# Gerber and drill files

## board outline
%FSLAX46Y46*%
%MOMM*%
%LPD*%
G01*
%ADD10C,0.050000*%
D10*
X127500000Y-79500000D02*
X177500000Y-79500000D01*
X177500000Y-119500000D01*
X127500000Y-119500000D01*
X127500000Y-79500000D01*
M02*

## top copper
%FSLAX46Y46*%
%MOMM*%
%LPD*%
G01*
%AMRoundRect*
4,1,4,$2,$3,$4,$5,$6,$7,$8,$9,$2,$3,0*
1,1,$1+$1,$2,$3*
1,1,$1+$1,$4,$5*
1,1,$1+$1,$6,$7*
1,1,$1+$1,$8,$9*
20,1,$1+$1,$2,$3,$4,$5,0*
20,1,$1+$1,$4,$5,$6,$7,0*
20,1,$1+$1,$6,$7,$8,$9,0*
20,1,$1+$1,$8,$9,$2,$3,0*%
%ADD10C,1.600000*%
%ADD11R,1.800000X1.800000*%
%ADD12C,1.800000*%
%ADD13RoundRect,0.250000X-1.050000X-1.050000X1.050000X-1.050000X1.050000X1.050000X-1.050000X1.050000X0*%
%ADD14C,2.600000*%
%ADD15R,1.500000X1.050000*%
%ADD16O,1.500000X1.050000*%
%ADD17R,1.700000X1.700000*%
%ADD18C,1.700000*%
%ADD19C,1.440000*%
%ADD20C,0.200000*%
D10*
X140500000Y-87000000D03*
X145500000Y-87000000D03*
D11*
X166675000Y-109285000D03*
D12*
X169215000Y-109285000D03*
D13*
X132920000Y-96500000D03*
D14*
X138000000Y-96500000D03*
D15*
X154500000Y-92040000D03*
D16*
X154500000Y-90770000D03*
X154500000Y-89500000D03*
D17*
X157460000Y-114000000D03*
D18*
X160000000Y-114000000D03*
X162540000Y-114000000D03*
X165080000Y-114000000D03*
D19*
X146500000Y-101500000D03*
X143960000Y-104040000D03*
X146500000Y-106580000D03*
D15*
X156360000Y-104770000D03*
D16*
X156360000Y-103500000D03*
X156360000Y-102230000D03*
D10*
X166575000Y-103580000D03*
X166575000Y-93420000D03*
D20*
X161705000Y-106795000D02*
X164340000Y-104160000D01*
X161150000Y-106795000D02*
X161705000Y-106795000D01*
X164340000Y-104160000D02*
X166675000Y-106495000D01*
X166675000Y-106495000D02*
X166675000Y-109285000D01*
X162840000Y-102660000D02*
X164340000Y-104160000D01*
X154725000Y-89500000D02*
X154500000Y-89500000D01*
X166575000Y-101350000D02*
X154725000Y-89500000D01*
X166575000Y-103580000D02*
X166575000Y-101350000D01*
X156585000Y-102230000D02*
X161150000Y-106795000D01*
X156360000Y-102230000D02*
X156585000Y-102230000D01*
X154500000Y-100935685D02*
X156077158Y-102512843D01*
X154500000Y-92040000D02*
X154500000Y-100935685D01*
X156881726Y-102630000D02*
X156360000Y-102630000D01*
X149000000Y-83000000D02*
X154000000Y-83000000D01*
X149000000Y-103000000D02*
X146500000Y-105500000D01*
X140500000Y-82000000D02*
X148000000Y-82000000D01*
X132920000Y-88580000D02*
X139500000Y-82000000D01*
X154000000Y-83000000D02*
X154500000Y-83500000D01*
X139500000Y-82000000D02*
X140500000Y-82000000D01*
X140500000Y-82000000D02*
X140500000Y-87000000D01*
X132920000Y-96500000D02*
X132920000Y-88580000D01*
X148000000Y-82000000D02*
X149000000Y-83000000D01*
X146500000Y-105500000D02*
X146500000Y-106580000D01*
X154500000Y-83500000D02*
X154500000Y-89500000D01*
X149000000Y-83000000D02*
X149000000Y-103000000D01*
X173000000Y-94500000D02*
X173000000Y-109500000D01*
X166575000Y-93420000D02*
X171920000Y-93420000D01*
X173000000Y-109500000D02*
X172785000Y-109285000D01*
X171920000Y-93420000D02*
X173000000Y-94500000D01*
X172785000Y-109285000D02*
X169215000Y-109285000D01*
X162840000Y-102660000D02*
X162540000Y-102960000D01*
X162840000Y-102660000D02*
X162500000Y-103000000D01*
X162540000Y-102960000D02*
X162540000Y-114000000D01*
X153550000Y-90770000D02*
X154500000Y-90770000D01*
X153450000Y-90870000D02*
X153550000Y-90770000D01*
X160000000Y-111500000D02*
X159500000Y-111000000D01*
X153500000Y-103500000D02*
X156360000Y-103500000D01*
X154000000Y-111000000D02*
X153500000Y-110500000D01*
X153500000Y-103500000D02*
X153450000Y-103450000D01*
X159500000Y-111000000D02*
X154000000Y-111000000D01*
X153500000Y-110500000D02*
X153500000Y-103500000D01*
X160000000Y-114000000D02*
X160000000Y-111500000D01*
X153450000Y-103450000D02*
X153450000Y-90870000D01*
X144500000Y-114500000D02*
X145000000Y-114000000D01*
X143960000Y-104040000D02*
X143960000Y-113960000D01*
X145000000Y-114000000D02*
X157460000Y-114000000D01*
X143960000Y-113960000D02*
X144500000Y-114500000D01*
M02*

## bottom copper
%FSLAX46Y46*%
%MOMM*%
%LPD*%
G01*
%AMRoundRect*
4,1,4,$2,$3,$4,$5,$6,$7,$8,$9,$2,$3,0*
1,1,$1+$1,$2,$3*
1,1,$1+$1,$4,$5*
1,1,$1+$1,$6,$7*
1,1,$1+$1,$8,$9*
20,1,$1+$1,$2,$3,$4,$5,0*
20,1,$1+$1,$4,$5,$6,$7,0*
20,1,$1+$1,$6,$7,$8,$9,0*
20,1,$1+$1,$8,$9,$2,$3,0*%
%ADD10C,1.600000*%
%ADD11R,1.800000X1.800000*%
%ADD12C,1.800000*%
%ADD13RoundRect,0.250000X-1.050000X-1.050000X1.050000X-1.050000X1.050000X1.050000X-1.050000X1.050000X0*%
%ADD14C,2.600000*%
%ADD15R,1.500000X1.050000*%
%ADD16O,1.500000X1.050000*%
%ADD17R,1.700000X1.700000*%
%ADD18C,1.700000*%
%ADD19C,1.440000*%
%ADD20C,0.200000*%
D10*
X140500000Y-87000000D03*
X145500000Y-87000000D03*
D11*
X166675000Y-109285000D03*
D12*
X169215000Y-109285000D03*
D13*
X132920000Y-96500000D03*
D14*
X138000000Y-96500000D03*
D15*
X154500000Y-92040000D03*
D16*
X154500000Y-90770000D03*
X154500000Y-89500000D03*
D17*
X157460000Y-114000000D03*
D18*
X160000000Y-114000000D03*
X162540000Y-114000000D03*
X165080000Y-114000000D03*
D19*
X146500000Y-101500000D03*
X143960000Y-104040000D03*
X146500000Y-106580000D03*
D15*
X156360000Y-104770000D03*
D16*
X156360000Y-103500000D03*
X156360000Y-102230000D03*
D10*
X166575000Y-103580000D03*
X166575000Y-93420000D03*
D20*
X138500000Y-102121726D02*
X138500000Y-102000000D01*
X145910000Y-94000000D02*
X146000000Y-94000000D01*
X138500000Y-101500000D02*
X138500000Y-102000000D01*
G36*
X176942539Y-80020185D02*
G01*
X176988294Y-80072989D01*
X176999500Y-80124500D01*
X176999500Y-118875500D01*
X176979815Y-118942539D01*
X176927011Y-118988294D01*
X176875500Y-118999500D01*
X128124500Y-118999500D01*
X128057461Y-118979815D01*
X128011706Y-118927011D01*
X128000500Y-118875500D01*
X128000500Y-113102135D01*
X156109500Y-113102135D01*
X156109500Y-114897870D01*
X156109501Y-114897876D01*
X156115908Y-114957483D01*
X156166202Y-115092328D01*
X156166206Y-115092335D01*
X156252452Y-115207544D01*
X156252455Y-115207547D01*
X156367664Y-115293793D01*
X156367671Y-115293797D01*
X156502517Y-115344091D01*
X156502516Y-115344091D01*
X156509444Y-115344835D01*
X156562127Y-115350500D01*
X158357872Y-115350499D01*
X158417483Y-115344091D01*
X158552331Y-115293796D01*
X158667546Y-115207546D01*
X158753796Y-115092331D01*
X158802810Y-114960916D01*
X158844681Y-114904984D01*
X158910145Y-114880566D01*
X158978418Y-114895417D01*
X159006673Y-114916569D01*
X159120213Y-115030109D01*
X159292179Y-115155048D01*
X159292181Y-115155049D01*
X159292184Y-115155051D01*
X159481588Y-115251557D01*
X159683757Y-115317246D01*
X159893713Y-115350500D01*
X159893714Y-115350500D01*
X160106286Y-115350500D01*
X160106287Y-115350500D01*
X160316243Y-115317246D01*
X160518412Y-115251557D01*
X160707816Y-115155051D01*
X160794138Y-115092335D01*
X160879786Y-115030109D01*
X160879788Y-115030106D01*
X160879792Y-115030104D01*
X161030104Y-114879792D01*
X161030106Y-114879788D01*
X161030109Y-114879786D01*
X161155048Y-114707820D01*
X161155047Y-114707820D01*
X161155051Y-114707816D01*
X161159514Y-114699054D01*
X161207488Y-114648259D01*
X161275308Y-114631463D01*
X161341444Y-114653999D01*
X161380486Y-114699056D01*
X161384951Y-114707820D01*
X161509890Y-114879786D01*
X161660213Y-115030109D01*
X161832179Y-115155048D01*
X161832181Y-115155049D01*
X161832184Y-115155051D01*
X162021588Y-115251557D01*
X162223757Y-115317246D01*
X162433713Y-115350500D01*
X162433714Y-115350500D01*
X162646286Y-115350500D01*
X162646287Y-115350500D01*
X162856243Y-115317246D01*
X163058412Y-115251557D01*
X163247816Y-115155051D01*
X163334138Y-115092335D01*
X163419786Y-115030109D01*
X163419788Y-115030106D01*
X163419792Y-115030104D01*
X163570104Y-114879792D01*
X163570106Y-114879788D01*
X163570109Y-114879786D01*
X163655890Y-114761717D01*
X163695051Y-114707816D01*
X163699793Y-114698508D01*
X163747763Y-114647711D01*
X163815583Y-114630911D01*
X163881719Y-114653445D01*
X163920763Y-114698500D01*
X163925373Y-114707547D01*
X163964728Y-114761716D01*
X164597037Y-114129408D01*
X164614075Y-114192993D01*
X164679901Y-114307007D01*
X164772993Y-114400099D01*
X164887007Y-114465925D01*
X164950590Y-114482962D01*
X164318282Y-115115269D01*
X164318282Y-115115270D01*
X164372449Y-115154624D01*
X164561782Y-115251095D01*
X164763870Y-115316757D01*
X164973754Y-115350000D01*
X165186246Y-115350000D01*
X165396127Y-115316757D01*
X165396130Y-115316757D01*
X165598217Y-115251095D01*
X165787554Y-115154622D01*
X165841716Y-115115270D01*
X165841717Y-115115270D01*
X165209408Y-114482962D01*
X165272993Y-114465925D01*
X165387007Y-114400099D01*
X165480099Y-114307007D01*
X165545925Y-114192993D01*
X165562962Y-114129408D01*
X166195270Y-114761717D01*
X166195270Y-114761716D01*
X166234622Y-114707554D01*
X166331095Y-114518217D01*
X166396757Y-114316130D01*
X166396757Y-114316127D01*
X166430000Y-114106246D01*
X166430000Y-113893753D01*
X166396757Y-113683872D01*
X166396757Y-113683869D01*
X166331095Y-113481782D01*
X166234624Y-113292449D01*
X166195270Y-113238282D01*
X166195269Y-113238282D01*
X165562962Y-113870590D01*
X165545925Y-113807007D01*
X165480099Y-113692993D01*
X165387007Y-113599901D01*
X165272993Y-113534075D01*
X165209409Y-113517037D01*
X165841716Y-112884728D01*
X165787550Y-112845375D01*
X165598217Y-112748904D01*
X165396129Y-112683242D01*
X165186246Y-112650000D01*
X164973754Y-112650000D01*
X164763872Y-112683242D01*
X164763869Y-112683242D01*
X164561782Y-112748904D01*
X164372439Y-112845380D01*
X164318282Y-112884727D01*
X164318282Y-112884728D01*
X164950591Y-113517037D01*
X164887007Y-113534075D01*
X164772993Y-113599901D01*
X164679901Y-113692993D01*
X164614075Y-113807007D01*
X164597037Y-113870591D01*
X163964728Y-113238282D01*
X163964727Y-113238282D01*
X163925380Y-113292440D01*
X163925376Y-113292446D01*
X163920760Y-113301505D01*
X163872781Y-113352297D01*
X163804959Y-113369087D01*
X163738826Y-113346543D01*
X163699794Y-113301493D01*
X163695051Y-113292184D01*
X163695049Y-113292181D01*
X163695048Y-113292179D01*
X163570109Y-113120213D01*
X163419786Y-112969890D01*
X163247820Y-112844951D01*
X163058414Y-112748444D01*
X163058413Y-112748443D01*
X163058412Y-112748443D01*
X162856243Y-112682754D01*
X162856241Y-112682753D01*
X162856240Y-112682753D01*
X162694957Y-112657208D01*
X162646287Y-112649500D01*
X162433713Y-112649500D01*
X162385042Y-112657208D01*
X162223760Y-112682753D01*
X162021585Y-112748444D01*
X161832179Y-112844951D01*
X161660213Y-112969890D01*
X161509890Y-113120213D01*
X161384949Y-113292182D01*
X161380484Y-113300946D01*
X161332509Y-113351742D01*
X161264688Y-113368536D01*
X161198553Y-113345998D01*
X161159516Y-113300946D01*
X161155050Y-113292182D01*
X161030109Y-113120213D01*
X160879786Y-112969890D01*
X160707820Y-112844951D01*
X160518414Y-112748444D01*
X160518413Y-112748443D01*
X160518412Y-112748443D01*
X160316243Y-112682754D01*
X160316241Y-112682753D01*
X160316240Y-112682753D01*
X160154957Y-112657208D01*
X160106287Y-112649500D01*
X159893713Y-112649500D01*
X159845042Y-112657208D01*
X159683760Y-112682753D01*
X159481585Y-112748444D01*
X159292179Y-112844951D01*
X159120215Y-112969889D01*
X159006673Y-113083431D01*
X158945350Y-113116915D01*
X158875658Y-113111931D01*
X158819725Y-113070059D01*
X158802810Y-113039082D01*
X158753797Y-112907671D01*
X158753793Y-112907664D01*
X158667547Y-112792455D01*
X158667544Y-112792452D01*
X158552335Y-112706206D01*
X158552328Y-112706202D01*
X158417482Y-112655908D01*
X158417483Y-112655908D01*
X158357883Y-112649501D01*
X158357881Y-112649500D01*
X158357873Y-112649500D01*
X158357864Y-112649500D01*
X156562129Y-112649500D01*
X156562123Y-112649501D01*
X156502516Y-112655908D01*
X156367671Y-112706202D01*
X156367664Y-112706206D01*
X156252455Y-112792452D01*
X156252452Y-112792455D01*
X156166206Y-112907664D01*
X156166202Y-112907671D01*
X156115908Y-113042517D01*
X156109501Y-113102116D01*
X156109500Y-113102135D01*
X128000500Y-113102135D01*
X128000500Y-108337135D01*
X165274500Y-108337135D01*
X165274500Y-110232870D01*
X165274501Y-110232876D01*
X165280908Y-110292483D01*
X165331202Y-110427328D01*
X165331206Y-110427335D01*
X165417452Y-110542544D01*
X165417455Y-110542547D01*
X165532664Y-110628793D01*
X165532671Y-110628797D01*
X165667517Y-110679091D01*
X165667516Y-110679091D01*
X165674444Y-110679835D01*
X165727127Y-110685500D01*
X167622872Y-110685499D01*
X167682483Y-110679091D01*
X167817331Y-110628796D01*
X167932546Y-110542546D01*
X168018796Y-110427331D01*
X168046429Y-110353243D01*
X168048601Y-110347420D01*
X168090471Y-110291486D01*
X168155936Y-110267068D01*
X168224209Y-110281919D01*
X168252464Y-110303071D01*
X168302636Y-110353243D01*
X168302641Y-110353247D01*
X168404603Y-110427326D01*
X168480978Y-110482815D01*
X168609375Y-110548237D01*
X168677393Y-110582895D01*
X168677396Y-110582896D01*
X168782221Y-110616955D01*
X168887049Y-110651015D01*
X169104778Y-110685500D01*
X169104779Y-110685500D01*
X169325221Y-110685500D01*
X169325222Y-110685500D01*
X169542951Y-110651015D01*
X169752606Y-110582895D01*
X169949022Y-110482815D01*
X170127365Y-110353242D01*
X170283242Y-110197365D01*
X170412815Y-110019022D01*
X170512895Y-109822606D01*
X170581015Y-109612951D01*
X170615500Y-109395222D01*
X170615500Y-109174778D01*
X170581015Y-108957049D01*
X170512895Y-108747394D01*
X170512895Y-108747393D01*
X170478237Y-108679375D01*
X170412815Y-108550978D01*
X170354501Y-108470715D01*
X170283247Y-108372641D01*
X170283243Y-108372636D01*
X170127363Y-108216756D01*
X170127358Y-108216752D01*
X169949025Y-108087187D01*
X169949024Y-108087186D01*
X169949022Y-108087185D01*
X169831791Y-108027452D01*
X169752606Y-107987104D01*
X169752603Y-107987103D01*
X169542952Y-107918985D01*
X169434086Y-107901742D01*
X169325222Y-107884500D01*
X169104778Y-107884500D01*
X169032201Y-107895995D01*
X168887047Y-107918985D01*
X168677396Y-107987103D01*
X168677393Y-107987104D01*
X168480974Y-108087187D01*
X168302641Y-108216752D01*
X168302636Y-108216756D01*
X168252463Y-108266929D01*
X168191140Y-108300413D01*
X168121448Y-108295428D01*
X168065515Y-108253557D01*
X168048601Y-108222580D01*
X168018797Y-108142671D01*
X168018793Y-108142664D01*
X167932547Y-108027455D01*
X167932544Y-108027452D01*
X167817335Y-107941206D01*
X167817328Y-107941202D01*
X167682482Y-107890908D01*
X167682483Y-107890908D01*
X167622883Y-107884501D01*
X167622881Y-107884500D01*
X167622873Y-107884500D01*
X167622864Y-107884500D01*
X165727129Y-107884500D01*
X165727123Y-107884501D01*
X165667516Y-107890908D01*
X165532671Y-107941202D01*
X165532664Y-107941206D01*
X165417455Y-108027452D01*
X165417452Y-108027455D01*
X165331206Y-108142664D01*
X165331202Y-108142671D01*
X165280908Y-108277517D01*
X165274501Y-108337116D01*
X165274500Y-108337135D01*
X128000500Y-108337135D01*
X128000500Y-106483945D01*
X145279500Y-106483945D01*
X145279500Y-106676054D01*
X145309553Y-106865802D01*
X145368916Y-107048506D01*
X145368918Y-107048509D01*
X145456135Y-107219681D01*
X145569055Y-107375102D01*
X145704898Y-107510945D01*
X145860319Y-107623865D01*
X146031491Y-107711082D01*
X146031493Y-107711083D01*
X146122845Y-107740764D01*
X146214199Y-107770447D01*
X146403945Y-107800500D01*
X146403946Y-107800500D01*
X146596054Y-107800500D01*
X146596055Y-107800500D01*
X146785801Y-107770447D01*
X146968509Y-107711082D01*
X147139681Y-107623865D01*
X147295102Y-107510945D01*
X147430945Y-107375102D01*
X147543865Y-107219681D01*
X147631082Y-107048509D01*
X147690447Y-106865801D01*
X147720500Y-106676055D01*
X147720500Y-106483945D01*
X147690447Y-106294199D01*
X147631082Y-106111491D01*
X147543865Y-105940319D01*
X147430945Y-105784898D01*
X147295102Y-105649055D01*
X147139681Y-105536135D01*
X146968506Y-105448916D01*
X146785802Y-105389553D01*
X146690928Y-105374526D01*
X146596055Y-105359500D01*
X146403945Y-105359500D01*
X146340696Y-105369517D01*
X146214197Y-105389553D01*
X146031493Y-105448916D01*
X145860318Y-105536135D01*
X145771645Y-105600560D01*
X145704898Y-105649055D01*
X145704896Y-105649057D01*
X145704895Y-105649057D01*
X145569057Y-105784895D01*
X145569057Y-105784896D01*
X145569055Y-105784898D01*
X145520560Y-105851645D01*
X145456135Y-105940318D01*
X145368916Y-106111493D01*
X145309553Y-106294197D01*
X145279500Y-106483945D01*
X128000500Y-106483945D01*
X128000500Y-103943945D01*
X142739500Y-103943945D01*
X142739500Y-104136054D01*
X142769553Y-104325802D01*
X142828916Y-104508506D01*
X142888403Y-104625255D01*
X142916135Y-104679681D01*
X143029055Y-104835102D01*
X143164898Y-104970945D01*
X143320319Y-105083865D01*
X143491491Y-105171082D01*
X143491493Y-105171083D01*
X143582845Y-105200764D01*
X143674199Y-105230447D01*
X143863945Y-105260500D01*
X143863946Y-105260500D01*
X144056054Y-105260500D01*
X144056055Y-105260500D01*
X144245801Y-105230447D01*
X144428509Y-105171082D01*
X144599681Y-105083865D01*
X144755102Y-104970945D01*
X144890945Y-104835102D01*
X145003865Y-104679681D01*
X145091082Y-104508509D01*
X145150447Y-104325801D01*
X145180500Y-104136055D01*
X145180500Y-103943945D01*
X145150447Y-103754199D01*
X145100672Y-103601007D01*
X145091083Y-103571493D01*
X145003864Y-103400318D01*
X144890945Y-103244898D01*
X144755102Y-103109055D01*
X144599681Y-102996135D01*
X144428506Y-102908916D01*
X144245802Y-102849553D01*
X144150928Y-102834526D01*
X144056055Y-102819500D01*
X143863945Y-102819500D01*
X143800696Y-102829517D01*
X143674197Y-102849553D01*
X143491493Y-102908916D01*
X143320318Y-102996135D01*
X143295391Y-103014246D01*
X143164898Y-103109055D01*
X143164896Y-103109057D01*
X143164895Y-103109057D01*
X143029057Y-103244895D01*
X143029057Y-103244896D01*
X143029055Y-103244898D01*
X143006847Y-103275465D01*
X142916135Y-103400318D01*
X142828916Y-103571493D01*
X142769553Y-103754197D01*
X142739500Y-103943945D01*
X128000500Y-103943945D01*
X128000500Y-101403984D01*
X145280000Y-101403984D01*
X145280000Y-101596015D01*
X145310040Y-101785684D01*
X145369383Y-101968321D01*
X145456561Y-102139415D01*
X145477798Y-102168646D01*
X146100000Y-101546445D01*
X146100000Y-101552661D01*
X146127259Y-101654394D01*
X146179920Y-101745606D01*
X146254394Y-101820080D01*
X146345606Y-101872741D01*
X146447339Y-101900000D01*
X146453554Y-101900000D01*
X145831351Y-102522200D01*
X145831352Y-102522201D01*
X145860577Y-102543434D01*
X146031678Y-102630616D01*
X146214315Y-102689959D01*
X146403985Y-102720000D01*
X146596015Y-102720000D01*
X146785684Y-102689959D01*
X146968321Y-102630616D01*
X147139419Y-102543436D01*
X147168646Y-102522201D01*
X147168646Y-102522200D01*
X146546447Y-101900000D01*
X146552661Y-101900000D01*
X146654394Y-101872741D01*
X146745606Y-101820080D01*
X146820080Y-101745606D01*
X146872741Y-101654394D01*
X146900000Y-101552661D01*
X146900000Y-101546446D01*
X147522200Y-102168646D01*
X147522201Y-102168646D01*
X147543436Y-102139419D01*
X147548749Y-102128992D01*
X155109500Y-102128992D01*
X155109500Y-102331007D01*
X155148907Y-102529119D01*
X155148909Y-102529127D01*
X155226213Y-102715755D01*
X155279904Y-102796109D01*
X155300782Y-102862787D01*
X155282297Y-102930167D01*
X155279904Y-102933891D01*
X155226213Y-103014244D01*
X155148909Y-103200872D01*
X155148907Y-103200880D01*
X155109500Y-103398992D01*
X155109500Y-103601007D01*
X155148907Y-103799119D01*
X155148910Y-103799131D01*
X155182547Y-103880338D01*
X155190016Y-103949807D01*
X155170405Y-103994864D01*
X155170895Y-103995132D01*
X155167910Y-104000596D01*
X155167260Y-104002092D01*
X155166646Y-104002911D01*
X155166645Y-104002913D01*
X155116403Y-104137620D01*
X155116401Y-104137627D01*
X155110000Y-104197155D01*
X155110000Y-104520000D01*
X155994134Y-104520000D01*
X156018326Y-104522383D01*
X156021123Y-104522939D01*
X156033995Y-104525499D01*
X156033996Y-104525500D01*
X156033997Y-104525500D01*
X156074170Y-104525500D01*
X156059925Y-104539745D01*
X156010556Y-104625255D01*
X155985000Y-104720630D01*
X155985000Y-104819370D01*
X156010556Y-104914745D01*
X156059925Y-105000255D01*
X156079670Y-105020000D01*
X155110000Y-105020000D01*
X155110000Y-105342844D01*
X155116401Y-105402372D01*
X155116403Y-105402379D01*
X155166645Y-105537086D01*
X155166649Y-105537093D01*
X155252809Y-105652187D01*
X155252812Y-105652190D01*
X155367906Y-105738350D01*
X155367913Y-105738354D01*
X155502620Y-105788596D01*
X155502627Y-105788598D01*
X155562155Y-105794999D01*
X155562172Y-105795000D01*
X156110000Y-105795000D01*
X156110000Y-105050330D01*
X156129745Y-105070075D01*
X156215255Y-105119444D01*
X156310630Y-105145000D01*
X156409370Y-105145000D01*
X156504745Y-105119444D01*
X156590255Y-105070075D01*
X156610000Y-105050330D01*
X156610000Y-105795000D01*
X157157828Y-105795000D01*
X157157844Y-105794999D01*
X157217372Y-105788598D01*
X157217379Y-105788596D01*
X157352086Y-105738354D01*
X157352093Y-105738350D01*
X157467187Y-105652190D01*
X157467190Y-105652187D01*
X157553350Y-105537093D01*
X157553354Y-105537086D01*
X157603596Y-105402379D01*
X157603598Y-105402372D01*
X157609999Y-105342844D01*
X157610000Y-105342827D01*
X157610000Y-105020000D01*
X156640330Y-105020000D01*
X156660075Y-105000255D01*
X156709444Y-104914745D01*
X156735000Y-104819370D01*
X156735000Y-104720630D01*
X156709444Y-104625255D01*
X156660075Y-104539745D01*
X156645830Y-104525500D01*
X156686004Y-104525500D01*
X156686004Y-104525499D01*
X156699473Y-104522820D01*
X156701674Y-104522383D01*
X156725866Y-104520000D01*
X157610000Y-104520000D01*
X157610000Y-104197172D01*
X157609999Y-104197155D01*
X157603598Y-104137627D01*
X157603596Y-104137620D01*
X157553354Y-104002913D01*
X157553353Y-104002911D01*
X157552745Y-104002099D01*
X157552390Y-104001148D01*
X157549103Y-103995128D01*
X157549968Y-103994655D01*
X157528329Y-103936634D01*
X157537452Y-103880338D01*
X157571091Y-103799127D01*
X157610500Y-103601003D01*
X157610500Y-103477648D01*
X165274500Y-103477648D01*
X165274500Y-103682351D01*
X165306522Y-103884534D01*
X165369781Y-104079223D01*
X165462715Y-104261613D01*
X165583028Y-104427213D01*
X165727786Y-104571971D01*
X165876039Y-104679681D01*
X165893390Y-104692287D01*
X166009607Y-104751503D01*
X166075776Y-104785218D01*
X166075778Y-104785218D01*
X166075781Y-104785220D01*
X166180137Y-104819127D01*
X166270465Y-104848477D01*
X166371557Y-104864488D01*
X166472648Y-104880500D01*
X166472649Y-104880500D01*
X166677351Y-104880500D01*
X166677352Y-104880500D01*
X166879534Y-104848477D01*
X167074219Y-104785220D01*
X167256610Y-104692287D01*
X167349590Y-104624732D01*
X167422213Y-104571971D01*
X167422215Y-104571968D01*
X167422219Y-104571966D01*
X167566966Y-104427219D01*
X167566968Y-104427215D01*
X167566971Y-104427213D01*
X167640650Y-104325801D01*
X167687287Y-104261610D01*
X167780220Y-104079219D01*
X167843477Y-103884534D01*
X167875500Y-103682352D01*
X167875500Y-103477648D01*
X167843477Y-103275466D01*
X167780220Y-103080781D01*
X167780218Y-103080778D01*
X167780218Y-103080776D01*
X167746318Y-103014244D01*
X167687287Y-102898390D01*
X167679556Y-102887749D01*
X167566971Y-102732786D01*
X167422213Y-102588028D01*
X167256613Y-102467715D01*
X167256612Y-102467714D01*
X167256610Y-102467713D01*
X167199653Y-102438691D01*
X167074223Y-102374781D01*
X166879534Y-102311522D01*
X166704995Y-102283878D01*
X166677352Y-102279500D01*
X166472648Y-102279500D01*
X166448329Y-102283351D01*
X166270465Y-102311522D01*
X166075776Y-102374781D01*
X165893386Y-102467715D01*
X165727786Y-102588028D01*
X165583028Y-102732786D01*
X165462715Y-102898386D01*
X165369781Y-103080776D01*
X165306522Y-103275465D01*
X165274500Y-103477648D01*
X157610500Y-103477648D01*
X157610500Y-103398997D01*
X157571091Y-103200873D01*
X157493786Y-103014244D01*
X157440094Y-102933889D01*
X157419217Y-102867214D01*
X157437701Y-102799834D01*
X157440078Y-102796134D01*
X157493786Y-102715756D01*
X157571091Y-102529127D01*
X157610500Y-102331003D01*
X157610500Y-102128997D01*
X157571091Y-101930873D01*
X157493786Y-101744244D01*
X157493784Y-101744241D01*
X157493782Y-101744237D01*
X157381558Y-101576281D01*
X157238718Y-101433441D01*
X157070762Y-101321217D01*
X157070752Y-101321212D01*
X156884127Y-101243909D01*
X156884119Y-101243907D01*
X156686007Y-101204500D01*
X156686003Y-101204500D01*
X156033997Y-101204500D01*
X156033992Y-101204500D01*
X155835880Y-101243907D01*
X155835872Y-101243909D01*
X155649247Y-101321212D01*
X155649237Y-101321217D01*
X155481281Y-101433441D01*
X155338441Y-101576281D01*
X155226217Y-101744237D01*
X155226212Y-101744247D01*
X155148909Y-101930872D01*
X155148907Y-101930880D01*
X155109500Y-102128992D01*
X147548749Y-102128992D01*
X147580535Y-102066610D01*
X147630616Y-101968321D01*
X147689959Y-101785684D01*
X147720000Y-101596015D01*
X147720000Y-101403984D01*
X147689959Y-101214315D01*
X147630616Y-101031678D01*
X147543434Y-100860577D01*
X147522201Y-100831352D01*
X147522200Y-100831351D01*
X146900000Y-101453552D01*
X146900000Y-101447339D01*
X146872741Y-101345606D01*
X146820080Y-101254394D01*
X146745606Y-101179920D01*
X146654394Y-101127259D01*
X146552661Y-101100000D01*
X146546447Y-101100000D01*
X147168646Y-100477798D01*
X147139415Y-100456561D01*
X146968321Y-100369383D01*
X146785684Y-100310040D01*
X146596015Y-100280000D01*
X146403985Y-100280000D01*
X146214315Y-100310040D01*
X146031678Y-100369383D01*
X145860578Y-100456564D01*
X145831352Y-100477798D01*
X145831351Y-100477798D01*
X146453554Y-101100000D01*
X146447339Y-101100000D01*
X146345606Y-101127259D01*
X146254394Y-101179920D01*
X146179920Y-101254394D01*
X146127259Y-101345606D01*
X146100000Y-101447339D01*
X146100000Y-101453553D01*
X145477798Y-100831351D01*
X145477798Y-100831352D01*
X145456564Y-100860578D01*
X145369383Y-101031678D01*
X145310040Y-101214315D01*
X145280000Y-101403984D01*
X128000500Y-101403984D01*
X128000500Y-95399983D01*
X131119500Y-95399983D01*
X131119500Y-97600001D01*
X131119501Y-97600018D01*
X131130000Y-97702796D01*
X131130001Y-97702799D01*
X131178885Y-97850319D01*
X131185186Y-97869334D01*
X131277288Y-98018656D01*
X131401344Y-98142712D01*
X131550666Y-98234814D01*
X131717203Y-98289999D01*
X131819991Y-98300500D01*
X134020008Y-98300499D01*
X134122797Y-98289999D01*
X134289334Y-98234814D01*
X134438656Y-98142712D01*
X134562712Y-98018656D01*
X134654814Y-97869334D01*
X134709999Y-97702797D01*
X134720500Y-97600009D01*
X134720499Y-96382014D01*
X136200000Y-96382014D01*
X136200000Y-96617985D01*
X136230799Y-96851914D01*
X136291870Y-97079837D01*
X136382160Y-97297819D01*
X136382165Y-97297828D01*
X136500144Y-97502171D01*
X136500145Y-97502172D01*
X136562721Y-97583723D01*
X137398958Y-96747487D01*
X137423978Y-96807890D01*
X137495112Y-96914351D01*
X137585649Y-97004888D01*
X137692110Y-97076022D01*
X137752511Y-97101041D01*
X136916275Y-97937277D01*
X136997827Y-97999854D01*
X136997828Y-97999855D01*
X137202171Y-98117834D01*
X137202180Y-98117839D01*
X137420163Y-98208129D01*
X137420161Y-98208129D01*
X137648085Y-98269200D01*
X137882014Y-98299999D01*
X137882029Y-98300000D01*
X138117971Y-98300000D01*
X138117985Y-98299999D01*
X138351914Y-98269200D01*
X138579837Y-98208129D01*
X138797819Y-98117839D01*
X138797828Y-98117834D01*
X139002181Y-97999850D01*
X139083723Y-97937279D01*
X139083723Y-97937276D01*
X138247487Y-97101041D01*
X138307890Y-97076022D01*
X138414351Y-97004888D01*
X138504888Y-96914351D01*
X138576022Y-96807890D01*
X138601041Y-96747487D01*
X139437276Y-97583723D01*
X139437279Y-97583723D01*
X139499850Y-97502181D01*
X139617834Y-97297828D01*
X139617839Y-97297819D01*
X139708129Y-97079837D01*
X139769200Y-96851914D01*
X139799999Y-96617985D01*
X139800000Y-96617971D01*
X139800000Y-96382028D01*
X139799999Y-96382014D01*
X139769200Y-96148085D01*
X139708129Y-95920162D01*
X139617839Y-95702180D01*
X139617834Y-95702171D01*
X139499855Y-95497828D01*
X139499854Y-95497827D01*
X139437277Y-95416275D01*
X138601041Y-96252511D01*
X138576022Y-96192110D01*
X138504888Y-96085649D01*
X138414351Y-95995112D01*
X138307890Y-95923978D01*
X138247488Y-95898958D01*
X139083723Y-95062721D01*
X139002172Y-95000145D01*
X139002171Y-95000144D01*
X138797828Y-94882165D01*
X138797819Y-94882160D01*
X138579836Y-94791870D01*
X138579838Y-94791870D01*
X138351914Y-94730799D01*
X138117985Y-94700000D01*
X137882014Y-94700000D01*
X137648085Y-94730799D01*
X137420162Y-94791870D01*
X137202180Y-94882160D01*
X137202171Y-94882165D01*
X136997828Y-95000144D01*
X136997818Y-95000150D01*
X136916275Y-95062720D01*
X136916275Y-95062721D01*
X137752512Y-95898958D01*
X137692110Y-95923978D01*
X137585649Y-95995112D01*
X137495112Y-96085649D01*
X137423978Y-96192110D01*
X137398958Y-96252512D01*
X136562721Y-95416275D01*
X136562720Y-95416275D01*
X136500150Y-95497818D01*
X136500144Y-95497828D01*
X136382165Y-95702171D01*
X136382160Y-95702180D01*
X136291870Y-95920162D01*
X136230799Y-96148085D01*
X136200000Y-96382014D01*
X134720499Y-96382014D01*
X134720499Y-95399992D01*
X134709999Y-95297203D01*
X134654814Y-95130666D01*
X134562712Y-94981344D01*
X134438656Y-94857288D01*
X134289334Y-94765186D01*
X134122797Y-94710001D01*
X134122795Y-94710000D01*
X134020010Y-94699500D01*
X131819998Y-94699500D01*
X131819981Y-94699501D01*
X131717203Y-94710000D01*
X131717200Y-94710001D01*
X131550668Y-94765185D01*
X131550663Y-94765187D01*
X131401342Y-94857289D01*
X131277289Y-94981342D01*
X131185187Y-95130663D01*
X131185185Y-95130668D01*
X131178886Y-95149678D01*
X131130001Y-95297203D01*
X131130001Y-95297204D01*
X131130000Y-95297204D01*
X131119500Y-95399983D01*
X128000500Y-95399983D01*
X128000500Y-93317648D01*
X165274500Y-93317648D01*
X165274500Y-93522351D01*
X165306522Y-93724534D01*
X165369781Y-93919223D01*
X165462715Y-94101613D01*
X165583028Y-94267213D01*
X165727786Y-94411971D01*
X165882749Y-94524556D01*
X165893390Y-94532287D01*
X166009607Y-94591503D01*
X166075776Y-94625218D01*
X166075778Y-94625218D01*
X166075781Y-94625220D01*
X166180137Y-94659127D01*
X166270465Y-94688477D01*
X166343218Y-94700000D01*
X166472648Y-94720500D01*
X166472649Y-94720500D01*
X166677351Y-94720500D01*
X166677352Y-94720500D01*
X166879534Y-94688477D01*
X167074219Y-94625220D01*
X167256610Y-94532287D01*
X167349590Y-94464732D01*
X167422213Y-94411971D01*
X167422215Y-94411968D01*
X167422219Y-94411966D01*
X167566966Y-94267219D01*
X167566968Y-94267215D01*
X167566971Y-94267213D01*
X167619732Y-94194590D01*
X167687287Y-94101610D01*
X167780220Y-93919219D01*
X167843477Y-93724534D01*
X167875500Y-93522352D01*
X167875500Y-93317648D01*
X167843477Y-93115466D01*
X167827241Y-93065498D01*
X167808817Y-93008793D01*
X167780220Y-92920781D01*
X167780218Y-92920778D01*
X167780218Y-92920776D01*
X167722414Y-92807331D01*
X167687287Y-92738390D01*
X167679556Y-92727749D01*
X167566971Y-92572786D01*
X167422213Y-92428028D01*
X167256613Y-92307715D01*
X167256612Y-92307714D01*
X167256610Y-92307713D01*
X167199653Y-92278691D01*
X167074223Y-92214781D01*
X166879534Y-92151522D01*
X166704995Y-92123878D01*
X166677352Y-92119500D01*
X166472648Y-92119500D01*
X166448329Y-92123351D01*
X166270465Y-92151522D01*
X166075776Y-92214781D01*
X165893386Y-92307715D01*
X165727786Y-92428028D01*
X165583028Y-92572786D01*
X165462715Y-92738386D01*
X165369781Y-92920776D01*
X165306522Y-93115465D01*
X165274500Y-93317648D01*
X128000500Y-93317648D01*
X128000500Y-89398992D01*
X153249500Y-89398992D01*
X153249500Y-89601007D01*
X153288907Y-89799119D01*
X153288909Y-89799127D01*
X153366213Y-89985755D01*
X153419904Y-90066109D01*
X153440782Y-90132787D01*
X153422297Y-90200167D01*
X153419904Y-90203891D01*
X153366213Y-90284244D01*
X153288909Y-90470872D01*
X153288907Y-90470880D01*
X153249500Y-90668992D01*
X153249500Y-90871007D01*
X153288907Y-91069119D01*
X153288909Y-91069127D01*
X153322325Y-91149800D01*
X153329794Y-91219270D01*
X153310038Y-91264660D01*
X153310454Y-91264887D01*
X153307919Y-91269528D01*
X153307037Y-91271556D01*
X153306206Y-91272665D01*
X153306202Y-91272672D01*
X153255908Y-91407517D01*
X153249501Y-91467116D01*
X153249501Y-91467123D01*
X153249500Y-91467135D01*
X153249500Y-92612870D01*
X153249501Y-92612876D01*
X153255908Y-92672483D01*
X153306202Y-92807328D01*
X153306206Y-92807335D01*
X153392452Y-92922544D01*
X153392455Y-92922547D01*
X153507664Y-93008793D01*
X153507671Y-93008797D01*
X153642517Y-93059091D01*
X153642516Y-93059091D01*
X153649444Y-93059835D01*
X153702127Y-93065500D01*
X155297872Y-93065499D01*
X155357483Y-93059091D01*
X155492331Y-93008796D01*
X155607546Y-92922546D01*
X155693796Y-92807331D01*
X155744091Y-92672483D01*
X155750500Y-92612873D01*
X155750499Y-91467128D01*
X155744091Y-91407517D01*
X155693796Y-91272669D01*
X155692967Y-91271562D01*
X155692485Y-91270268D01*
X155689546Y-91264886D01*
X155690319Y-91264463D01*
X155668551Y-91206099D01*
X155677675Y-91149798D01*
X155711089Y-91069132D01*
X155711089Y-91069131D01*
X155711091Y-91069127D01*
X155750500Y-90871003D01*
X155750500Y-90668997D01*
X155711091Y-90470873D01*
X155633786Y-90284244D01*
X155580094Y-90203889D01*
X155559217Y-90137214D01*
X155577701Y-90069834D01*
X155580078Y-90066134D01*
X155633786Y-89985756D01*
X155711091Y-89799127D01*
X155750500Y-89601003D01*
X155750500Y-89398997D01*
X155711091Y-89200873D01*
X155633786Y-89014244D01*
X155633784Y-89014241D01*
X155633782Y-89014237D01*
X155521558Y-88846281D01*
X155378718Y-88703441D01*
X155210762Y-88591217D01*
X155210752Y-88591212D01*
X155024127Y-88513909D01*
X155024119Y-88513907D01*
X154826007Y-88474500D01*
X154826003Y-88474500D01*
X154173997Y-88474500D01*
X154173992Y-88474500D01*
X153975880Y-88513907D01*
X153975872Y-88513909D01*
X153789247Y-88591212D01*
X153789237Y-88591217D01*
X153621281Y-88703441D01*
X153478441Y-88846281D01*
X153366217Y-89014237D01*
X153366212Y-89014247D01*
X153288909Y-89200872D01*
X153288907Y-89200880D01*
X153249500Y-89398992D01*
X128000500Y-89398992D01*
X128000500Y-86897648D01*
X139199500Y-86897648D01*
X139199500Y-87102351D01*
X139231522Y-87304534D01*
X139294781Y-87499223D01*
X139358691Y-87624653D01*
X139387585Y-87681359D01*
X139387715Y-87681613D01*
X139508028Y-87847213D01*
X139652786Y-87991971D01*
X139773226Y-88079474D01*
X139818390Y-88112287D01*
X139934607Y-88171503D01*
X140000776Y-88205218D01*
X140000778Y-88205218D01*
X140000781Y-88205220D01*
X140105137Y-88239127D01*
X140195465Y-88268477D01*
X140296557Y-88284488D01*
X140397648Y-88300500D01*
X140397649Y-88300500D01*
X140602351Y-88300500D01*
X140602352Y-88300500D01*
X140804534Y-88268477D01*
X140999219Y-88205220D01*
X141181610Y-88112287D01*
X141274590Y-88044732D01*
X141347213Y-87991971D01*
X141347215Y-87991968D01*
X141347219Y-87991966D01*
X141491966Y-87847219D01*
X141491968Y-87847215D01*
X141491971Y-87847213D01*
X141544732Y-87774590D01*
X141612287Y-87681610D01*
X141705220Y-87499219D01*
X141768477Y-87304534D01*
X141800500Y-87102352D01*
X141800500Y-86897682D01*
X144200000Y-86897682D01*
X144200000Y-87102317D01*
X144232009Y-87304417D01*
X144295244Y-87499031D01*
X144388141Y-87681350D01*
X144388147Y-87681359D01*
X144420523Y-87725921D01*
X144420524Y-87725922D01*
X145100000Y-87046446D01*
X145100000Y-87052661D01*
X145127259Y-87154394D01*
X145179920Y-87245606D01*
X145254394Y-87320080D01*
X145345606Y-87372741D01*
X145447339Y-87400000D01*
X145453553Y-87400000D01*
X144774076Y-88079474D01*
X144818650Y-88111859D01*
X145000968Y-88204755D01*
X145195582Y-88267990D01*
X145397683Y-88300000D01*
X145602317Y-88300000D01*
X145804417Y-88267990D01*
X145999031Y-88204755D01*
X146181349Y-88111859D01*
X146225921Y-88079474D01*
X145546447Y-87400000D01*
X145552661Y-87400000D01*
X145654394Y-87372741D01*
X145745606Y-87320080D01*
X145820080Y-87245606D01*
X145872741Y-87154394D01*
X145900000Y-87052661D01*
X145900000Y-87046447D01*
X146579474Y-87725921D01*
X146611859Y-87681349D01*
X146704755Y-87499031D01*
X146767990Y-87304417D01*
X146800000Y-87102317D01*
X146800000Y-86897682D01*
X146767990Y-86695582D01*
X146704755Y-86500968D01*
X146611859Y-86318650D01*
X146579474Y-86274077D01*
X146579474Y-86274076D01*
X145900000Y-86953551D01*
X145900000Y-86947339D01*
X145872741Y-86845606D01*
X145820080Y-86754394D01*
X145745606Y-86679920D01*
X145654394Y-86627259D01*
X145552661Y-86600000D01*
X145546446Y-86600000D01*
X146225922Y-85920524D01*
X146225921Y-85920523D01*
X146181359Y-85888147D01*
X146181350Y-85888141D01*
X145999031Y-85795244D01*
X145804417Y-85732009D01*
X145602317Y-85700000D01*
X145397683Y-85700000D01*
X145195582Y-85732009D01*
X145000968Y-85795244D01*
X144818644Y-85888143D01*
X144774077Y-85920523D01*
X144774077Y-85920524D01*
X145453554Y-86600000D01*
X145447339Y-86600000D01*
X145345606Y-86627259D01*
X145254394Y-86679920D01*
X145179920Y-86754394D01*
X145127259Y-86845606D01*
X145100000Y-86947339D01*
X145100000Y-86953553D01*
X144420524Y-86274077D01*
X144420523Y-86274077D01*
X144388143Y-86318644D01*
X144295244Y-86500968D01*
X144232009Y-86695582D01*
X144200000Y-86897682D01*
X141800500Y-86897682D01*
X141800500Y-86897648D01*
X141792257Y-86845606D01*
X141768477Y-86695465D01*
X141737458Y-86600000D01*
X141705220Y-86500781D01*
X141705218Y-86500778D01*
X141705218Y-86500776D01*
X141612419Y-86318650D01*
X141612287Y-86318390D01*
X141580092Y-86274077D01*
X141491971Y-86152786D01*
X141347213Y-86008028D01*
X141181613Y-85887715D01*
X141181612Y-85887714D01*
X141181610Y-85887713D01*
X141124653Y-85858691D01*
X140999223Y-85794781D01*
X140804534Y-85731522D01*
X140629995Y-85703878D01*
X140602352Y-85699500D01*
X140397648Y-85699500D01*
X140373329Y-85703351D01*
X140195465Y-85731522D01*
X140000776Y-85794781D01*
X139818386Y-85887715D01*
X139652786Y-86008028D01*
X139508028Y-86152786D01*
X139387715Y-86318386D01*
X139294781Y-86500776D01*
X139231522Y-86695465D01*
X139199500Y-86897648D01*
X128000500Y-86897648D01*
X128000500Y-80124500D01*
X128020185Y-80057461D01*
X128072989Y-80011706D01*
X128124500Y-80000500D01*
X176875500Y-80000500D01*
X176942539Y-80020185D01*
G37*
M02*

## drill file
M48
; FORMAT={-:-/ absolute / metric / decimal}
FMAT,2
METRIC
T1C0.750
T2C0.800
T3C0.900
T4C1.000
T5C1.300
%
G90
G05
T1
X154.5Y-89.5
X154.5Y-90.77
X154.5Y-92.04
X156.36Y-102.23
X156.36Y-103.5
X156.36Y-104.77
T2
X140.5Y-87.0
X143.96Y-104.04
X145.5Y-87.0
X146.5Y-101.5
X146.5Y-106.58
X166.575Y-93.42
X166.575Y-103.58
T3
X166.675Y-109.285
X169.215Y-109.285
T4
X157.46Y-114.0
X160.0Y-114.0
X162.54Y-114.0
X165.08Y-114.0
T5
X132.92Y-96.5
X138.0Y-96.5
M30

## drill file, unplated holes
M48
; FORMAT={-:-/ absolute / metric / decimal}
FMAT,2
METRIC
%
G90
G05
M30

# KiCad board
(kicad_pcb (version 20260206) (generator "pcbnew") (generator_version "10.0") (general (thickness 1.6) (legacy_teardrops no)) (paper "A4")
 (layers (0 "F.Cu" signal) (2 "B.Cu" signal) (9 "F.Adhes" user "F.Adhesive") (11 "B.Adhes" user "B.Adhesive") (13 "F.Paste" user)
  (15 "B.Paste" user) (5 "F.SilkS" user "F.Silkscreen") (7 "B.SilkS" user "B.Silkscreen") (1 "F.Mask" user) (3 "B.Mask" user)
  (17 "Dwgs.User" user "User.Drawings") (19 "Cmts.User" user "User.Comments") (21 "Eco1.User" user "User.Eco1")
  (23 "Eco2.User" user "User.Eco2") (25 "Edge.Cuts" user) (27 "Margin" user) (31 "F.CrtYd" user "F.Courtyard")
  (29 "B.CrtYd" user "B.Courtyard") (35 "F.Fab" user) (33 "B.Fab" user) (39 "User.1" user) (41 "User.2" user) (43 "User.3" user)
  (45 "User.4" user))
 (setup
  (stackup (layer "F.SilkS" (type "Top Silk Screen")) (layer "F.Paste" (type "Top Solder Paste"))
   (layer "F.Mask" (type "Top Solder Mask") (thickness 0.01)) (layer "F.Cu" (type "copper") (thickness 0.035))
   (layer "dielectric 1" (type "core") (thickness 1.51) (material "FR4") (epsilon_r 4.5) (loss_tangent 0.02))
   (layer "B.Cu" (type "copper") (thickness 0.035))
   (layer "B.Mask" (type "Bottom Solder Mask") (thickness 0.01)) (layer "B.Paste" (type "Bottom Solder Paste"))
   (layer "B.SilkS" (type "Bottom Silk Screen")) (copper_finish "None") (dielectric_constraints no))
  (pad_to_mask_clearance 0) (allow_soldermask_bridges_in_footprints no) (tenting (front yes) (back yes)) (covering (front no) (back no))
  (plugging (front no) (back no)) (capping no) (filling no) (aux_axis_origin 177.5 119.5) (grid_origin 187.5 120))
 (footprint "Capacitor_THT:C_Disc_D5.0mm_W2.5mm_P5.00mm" (layer "F.Cu") (at 140.5 87)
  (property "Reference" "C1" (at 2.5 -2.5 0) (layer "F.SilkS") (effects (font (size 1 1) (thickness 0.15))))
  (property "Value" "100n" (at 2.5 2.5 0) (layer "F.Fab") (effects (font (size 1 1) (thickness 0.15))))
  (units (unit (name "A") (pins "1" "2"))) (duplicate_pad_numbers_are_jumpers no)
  (pad "1" thru_hole circle (at 0 0) (size 1.6 1.6) (drill 0.8) (layers "*.Cu" "*.Mask") (remove_unused_layers no) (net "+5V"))
  (pad "2" thru_hole circle (at 5 0) (size 1.6 1.6) (drill 0.8) (layers "*.Cu" "*.Mask") (remove_unused_layers no) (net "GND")))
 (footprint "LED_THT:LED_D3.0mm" (layer "F.Cu") (at 166.675 109.285)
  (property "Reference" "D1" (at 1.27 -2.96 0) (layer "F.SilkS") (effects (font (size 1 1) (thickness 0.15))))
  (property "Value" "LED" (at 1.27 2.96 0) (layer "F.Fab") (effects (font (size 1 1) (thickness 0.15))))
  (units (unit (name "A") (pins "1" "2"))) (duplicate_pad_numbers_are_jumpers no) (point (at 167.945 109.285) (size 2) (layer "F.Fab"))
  (pad "1" thru_hole rect (at 0 0) (size 1.8 1.8) (drill 0.9) (layers "*.Cu" "*.Mask") (remove_unused_layers no) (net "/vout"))
  (pad "2" thru_hole circle (at 2.54 0) (size 1.8 1.8) (drill 0.9) (layers "*.Cu" "*.Mask") (remove_unused_layers no) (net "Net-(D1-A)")))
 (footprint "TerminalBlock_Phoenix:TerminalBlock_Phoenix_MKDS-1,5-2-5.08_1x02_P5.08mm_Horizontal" (layer "F.Cu") (at 132.92 96.5)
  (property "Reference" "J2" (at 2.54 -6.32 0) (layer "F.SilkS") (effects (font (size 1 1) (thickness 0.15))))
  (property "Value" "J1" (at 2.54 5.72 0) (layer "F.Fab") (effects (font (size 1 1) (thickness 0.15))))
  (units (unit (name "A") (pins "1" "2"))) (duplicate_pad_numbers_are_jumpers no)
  (pad "1" thru_hole roundrect (at 0 0) (size 2.6 2.6) (drill 1.3) (layers "*.Cu" "*.Mask") (remove_unused_layers no)
   (roundrect_rratio 0.096154) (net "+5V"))
  (pad "2" thru_hole circle (at 5.08 0) (size 2.6 2.6) (drill 1.3) (layers "*.Cu" "*.Mask") (remove_unused_layers no) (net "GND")))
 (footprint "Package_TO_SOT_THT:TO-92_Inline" (layer "F.Cu") (at 154.5 92.04 90)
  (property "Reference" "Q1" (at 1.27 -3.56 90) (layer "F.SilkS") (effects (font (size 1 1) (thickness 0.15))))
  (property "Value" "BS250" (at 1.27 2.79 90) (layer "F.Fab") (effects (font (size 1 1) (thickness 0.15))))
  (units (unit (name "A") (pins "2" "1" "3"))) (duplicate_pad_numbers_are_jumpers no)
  (pad "1" thru_hole rect (at 0 0 90) (size 1.05 1.5) (drill 0.75) (layers "*.Cu" "*.Mask") (remove_unused_layers no) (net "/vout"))
  (pad "2" thru_hole oval (at 1.27 0 90) (size 1.05 1.5) (drill 0.75) (layers "*.Cu" "*.Mask") (remove_unused_layers no) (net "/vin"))
  (pad "3" thru_hole oval (at 2.54 0 90) (size 1.05 1.5) (drill 0.75) (layers "*.Cu" "*.Mask") (remove_unused_layers no) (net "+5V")))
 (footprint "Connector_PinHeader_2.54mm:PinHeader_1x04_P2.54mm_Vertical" (layer "F.Cu") (at 157.46 114 90)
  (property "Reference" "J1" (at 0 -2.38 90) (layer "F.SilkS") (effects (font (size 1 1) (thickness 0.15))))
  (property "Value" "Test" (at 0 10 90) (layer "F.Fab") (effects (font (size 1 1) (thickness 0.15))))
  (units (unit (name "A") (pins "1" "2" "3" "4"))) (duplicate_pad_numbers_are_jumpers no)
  (pad "1" thru_hole rect (at 0 0 90) (size 1.7 1.7) (drill 1) (layers "*.Cu" "*.Mask") (remove_unused_layers no) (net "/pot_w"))
  (pad "2" thru_hole circle (at 0 2.54 90) (size 1.7 1.7) (drill 1) (layers "*.Cu" "*.Mask") (remove_unused_layers no) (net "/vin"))
  (pad "3" thru_hole circle (at 0 5.08 90) (size 1.7 1.7) (drill 1) (layers "*.Cu" "*.Mask") (remove_unused_layers no) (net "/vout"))
  (pad "4" thru_hole circle (at 0 7.62 90) (size 1.7 1.7) (drill 1) (layers "*.Cu" "*.Mask") (remove_unused_layers no) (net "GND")))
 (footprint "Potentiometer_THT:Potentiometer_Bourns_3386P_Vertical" (layer "F.Cu") (at 146.5 101.5 180)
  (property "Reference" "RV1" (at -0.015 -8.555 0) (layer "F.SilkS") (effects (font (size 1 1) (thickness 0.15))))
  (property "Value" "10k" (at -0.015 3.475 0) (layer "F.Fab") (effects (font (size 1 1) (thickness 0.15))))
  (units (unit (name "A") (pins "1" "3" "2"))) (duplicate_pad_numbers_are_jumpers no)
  (pad "1" thru_hole circle (at 0 0 180) (size 1.44 1.44) (drill 0.8) (layers "*.Cu" "*.Mask") (remove_unused_layers no) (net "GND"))
  (pad "2" thru_hole circle (at 2.54 -2.54 180) (size 1.44 1.44) (drill 0.8) (layers "*.Cu" "*.Mask") (remove_unused_layers no)
   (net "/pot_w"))
  (pad "3" thru_hole circle (at 0 -5.08 180) (size 1.44 1.44) (drill 0.8) (layers "*.Cu" "*.Mask") (remove_unused_layers no) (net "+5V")))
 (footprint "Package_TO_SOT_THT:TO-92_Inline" (layer "F.Cu") (at 156.36 104.77 90)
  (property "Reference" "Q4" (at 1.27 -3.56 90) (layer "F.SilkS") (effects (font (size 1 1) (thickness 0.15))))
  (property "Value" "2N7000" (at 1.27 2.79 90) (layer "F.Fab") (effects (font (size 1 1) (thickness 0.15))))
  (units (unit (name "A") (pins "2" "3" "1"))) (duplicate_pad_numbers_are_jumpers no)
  (pad "1" thru_hole rect (at 0 0 90) (size 1.05 1.5) (drill 0.75) (layers "*.Cu" "*.Mask") (remove_unused_layers no) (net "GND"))
  (pad "2" thru_hole oval (at 1.27 0 90) (size 1.05 1.5) (drill 0.75) (layers "*.Cu" "*.Mask") (remove_unused_layers no) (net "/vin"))
  (pad "3" thru_hole oval (at 2.54 0 90) (size 1.05 1.5) (drill 0.75) (layers "*.Cu" "*.Mask") (remove_unused_layers no) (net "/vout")))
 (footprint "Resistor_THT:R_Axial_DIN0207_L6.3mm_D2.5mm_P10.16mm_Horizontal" (layer "F.Cu") (at 166.575 103.58 90)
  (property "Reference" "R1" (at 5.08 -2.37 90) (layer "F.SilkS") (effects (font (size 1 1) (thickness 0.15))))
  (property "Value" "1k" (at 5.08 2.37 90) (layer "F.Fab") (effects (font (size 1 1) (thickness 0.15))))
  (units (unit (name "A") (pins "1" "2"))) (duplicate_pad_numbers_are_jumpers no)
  (pad "1" thru_hole circle (at 0 0 90) (size 1.6 1.6) (drill 0.8) (layers "*.Cu" "*.Mask") (remove_unused_layers no) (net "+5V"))
  (pad "2" thru_hole circle (at 10.16 0 90) (size 1.6 1.6) (drill 0.8) (layers "*.Cu" "*.Mask") (remove_unused_layers no) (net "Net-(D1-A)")))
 (gr_rect (start 127.5 79.5) (end 177.5 119.5) (stroke (width 0.05) (type default)) (fill no) (layer "Edge.Cuts"))
 (segment (start 149 83) (end 154 83) (width 0.2) (layer "F.Cu") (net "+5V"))
 (segment (start 149 103) (end 146.5 105.5) (width 0.2) (layer "F.Cu") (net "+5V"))
 (segment (start 140.5 82) (end 148 82) (width 0.2) (layer "F.Cu") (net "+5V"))
 (segment (start 166.575 103.58) (end 166.575 101.35) (width 0.2) (layer "F.Cu") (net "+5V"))
 (segment (start 132.92 88.58) (end 139.5 82) (width 0.2) (layer "F.Cu") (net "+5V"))
 (segment (start 154 83) (end 154.5 83.5) (width 0.2) (layer "F.Cu") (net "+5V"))
 (segment (start 154.725 89.5) (end 154.5 89.5) (width 0.2) (layer "F.Cu") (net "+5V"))
 (segment (start 139.5 82) (end 140.5 82) (width 0.2) (layer "F.Cu") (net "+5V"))
 (segment (start 140.5 82) (end 140.5 87) (width 0.2) (layer "F.Cu") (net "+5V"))
 (segment (start 132.92 96.5) (end 132.92 88.58) (width 0.2) (layer "F.Cu") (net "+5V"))
 (segment (start 148 82) (end 149 83) (width 0.2) (layer "F.Cu") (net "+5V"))
 (segment (start 146.5 105.5) (end 146.5 106.58) (width 0.2) (layer "F.Cu") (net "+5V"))
 (segment (start 154.5 83.5) (end 154.5 89.5) (width 0.2) (layer "F.Cu") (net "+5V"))
 (segment (start 149 83) (end 149 103) (width 0.2) (layer "F.Cu") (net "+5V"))
 (segment (start 166.575 101.35) (end 154.725 89.5) (width 0.2) (layer "F.Cu") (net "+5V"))
 (segment (start 138.5 102.121726) (end 138.5 102) (width 0.2) (layer "B.Cu") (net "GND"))
 (segment (start 145.91 94) (end 146 94) (width 0.2) (layer "B.Cu") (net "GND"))
 (segment (start 138.5 101.5) (end 138.5 102) (width 0.2) (layer "B.Cu") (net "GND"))
 (segment (start 173 94.5) (end 173 109.5) (width 0.2) (layer "F.Cu") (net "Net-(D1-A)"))
 (segment (start 166.575 93.42) (end 171.92 93.42) (width 0.2) (layer "F.Cu") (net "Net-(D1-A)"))
 (segment (start 173 109.5) (end 172.785 109.285) (width 0.2) (layer "F.Cu") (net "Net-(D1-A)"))
 (segment (start 171.92 93.42) (end 173 94.5) (width 0.2) (layer "F.Cu") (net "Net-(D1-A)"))
 (segment (start 172.785 109.285) (end 169.215 109.285) (width 0.2) (layer "F.Cu") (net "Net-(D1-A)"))
 (segment (start 166.675 106.495) (end 166.675 109.285) (width 0.2) (layer "F.Cu") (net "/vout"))
 (segment (start 161.15 106.795) (end 161.705 106.795) (width 0.2) (layer "F.Cu") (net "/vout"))
 (segment (start 154.5 92.04) (end 154.5 100.935685) (width 0.2) (layer "F.Cu") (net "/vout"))
 (segment (start 156.585 102.23) (end 161.15 106.795) (width 0.2) (layer "F.Cu") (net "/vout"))
 (segment (start 162.84 102.66) (end 162.54 102.96) (width 0.2) (layer "F.Cu") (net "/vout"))
 (segment (start 164.34 104.16) (end 166.675 106.495) (width 0.2) (layer "F.Cu") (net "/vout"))
 (segment (start 154.5 100.935685) (end 156.077158 102.512843) (width 0.2) (layer "F.Cu") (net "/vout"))
 (segment (start 162.84 102.66) (end 162.5 103) (width 0.2) (layer "F.Cu") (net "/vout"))
 (segment (start 162.84 102.66) (end 164.34 104.16) (width 0.2) (layer "F.Cu") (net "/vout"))
 (segment (start 156.881726 102.63) (end 156.36 102.63) (width 0.2) (layer "F.Cu") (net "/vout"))
 (segment (start 156.36 102.23) (end 156.585 102.23) (width 0.2) (layer "F.Cu") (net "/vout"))
 (segment (start 162.54 102.96) (end 162.54 114) (width 0.2) (layer "F.Cu") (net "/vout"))
 (segment (start 161.705 106.795) (end 164.34 104.16) (width 0.2) (layer "F.Cu") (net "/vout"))
 (segment (start 153.55 90.77) (end 154.5 90.77) (width 0.2) (layer "F.Cu") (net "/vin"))
 (segment (start 153.45 90.87) (end 153.55 90.77) (width 0.2) (layer "F.Cu") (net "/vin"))
 (segment (start 160 111.5) (end 159.5 111) (width 0.2) (layer "F.Cu") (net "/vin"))
 (segment (start 153.5 103.5) (end 156.36 103.5) (width 0.2) (layer "F.Cu") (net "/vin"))
 (segment (start 154 111) (end 153.5 110.5) (width 0.2) (layer "F.Cu") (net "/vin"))
 (segment (start 153.5 103.5) (end 153.45 103.45) (width 0.2) (layer "F.Cu") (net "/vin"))
 (segment (start 159.5 111) (end 154 111) (width 0.2) (layer "F.Cu") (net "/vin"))
 (segment (start 153.5 110.5) (end 153.5 103.5) (width 0.2) (layer "F.Cu") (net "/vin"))
 (segment (start 160 114) (end 160 111.5) (width 0.2) (layer "F.Cu") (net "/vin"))
 (segment (start 153.45 103.45) (end 153.45 90.87) (width 0.2) (layer "F.Cu") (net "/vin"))
 (segment (start 144.5 114.5) (end 145 114) (width 0.2) (layer "F.Cu") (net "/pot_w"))
 (segment (start 143.96 104.04) (end 143.96 113.96) (width 0.2) (layer "F.Cu") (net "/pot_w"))
 (segment (start 145 114) (end 157.46 114) (width 0.2) (layer "F.Cu") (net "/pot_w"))
 (segment (start 143.96 113.96) (end 144.5 114.5) (width 0.2) (layer "F.Cu") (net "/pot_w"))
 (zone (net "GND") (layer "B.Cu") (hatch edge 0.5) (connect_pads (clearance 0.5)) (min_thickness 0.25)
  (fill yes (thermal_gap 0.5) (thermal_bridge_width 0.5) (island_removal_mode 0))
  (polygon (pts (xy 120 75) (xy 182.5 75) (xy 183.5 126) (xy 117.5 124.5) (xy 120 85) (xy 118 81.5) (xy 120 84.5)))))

